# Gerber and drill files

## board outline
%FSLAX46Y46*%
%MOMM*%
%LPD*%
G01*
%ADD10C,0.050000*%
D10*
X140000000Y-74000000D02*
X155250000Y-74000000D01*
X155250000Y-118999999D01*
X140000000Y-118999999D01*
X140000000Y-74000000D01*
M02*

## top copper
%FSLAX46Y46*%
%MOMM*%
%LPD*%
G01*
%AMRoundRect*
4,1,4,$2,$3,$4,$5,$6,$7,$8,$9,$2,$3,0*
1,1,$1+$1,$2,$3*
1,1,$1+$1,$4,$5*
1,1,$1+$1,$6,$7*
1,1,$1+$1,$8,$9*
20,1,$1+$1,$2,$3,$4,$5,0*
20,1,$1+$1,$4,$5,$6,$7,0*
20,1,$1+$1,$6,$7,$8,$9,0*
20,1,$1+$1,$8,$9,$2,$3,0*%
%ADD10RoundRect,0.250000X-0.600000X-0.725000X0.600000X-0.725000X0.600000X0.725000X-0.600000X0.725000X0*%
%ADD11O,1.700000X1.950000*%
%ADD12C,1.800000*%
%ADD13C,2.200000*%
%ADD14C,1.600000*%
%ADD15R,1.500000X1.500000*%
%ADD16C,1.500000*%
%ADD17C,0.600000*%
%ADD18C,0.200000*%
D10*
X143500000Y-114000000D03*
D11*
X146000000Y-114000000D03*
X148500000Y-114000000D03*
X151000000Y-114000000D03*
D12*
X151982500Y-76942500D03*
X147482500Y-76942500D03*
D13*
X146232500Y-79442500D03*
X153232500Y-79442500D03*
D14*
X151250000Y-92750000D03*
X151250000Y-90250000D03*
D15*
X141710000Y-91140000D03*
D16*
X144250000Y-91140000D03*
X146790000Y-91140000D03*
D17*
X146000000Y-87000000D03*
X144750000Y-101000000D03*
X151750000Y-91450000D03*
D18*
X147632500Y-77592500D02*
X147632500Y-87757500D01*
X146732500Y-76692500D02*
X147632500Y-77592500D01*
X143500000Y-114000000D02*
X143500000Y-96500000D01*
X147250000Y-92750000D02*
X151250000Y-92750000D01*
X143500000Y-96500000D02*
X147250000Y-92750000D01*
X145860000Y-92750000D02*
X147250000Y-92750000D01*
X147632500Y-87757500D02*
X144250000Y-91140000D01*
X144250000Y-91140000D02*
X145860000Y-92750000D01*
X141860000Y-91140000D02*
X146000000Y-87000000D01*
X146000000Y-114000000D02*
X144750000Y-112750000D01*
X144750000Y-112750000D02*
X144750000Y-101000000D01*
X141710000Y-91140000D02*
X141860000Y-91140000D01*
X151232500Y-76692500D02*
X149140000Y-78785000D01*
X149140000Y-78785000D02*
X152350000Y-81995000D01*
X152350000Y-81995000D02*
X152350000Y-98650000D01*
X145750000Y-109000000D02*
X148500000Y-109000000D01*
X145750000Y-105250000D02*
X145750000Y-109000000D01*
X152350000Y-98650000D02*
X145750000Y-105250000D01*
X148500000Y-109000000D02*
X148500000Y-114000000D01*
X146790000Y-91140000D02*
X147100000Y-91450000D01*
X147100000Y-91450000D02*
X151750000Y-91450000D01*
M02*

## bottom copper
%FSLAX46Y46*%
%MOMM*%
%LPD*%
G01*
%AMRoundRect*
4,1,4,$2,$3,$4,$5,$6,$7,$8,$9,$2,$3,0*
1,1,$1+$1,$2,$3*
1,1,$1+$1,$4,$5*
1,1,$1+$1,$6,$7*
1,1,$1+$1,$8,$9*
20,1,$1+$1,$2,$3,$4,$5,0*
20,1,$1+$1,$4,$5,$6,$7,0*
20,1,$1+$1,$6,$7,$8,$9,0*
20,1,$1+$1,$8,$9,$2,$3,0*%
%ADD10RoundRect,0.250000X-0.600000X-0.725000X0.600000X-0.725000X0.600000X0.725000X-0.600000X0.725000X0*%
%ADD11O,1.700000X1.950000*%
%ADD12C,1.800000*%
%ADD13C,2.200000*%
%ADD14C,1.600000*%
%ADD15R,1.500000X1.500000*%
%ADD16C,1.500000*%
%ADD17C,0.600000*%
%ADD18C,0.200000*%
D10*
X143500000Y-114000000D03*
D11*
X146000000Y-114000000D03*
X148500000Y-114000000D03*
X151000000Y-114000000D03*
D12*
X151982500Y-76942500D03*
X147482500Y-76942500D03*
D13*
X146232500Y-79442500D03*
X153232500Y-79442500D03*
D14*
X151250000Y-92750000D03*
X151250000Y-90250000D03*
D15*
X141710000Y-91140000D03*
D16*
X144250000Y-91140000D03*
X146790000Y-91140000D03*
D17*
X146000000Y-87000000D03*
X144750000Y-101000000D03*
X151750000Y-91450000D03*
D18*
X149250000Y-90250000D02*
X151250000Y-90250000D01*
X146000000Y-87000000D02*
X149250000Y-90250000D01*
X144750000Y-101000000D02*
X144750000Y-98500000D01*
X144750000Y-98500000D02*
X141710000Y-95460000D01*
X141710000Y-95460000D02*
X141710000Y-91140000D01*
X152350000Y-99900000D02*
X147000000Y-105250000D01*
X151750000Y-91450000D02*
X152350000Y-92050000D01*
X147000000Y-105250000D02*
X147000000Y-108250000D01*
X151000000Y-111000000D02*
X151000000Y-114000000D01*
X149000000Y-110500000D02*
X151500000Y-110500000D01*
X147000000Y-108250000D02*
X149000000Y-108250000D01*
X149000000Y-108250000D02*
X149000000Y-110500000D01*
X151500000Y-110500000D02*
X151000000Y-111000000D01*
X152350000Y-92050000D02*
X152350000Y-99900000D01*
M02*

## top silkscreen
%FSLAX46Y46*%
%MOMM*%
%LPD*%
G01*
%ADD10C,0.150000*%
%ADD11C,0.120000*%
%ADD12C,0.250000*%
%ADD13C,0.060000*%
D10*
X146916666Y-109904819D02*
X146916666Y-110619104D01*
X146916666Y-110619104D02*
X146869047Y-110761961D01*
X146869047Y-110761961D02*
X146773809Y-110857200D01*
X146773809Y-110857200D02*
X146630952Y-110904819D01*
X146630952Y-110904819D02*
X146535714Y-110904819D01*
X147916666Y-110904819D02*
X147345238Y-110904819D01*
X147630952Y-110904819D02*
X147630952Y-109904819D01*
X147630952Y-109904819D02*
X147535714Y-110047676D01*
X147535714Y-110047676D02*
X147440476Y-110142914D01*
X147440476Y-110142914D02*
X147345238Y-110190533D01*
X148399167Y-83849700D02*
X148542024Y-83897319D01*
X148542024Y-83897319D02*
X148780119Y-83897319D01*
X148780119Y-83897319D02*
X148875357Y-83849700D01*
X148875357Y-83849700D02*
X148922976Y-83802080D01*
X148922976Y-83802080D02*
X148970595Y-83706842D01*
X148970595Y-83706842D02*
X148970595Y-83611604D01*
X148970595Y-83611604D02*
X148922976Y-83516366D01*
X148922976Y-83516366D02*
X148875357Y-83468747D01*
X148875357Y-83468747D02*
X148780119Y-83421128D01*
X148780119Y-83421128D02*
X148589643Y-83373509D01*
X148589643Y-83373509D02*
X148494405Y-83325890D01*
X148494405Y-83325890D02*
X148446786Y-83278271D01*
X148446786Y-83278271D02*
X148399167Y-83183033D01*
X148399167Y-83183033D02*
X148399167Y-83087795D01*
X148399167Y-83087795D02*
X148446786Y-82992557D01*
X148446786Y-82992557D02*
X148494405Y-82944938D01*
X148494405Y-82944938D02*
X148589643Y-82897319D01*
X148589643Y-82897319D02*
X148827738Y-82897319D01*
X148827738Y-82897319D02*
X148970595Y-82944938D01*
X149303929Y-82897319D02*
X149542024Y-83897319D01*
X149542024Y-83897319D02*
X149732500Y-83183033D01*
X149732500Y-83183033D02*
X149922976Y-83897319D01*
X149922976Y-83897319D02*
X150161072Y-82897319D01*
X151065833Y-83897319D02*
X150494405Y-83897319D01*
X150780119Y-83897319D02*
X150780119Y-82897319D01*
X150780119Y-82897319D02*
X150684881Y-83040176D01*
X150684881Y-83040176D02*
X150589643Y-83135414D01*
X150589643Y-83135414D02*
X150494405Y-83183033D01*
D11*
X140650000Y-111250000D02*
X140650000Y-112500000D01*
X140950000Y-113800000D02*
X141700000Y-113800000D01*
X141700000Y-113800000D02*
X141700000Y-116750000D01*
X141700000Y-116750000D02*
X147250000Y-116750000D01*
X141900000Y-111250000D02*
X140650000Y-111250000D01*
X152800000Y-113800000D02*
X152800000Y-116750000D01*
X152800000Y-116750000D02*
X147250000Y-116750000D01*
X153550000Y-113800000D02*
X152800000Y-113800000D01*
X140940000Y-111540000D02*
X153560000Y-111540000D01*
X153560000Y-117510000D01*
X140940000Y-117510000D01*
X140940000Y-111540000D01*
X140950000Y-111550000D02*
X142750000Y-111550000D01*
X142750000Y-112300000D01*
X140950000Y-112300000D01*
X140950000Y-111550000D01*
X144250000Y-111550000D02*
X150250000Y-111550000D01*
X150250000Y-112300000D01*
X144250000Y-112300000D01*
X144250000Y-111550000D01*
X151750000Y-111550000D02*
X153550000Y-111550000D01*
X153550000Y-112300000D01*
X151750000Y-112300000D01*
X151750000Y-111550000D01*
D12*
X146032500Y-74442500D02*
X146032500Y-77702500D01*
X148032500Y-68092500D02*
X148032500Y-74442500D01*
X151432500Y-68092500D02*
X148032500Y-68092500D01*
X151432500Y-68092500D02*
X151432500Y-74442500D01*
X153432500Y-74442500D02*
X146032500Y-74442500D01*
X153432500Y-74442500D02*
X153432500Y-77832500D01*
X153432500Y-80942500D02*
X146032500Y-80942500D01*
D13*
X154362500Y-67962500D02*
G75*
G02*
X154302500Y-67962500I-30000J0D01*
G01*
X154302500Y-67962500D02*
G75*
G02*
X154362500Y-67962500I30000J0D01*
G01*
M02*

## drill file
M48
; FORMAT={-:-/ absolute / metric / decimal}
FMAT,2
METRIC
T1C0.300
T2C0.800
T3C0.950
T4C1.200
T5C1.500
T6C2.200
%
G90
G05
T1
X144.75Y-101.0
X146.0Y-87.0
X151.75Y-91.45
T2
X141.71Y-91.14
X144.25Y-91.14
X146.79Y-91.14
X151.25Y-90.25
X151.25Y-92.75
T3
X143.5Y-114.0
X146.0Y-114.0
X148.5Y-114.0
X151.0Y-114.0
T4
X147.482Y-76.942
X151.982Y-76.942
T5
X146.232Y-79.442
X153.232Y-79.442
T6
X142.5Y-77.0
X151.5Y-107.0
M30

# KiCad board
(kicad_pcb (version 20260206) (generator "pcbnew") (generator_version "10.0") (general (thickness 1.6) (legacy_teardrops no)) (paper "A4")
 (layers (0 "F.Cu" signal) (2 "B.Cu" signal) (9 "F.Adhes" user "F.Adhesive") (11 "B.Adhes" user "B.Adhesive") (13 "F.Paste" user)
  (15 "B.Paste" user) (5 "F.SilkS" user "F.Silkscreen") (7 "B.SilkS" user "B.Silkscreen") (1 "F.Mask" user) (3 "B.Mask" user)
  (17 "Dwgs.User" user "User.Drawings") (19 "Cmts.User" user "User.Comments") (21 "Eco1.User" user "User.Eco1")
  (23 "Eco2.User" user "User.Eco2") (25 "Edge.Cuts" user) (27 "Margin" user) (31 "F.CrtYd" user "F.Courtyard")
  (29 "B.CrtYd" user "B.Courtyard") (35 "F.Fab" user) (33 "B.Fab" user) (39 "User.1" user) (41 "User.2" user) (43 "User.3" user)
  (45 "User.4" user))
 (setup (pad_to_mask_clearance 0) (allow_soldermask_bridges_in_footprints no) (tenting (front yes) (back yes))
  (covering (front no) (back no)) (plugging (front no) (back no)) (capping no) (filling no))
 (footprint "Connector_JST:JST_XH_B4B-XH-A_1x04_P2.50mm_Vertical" (layer "F.Cu") (at 143.5 114)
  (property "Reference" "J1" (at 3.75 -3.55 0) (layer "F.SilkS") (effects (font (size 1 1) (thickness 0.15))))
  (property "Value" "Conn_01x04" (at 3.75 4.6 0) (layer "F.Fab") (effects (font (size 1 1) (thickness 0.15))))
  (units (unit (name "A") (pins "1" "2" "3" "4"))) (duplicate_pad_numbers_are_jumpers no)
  (fp_line (start -2.85 -2.75) (end -2.85 -1.5) (stroke (width 0.12) (type solid)) (layer "F.SilkS"))
  (fp_line (start -2.55 -0.2) (end -1.8 -0.2) (stroke (width 0.12) (type solid)) (layer "F.SilkS"))
  (fp_line (start -1.8 -0.2) (end -1.8 2.75) (stroke (width 0.12) (type solid)) (layer "F.SilkS"))
  (fp_line (start -1.8 2.75) (end 3.75 2.75) (stroke (width 0.12) (type solid)) (layer "F.SilkS"))
  (fp_line (start -1.6 -2.75) (end -2.85 -2.75) (stroke (width 0.12) (type solid)) (layer "F.SilkS"))
  (fp_line (start 9.3 -0.2) (end 9.3 2.75) (stroke (width 0.12) (type solid)) (layer "F.SilkS"))
  (fp_line (start 9.3 2.75) (end 3.75 2.75) (stroke (width 0.12) (type solid)) (layer "F.SilkS"))
  (fp_line (start 10.05 -0.2) (end 9.3 -0.2) (stroke (width 0.12) (type solid)) (layer "F.SilkS"))
  (fp_rect (start -2.56 -2.46) (end 10.06 3.51) (stroke (width 0.12) (type solid)) (fill no) (layer "F.SilkS"))
  (fp_rect (start -2.55 -2.45) (end -0.75 -1.7) (stroke (width 0.12) (type solid)) (fill no) (layer "F.SilkS"))
  (fp_rect (start 0.75 -2.45) (end 6.75 -1.7) (stroke (width 0.12) (type solid)) (fill no) (layer "F.SilkS"))
  (fp_rect (start 8.25 -2.45) (end 10.05 -1.7) (stroke (width 0.12) (type solid)) (fill no) (layer "F.SilkS"))
  (pad "1" thru_hole roundrect (at 0 0) (size 1.7 1.95) (drill 0.95) (layers "*.Cu" "*.Mask") (remove_unused_layers no)
   (roundrect_rratio 0.147059) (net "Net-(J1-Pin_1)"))
  (pad "2" thru_hole oval (at 2.5 0) (size 1.7 1.95) (drill 0.95) (layers "*.Cu" "*.Mask") (remove_unused_layers no) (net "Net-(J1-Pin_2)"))
  (pad "3" thru_hole oval (at 5 0) (size 1.7 1.95) (drill 0.95) (layers "*.Cu" "*.Mask") (remove_unused_layers no) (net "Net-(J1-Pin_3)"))
  (pad "4" thru_hole oval (at 7.5 0) (size 1.7 1.95) (drill 0.95) (layers "*.Cu" "*.Mask") (remove_unused_layers no) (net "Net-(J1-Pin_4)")))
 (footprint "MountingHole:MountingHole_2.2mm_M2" (layer "F.Cu") (at 142.5 77)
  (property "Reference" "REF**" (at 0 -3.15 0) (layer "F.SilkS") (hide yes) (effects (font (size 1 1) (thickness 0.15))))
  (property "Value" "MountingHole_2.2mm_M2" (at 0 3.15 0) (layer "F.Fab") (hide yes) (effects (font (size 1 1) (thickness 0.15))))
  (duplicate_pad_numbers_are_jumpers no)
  (pad "" np_thru_hole circle (at 0 0) (size 2.2 2.2) (drill 2.2) (layers "*.Cu" "*.Mask")))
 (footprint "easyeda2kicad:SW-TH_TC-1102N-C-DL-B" (layer "F.Cu") (at 149.7325 78.1925 180)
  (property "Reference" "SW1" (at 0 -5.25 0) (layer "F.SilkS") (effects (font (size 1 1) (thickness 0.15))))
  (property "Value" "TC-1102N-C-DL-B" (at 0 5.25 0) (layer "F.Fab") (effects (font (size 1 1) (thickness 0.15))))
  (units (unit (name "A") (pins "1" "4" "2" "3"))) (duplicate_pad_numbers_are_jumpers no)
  (fp_line (start 3.7 3.75) (end 3.7 0.49) (stroke (width 0.25) (type solid)) (layer "F.SilkS"))
  (fp_line (start 1.7 10.1) (end 1.7 3.75) (stroke (width 0.25) (type solid)) (layer "F.SilkS"))
  (fp_line (start -1.7 10.1) (end 1.7 10.1) (stroke (width 0.25) (type solid)) (layer "F.SilkS"))
  (fp_line (start -1.7 10.1) (end -1.7 3.75) (stroke (width 0.25) (type solid)) (layer "F.SilkS"))
  (fp_line (start -3.7 3.75) (end 3.7 3.75) (stroke (width 0.25) (type solid)) (layer "F.SilkS"))
  (fp_line (start -3.7 3.75) (end -3.7 0.36) (stroke (width 0.25) (type solid)) (layer "F.SilkS"))
  (fp_line (start -3.7 -2.75) (end 3.7 -2.75) (stroke (width 0.25) (type solid)) (layer "F.SilkS"))
  (fp_circle (center -4.6 10.23) (end -4.57 10.23) (stroke (width 0.06) (type solid)) (fill no) (layer "F.SilkS"))
  (pad "1" thru_hole circle (at -2.25 1.25 180) (size 1.8 1.8) (drill 1.199998) (layers "*.Cu" "*.Mask") (remove_unused_layers no)
   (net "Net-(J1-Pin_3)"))
  (pad "2" thru_hole circle (at 2.25 1.25 180) (size 1.8 1.8) (drill 1.199998) (layers "*.Cu" "*.Mask") (remove_unused_layers no)
   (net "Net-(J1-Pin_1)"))
  (pad "3" thru_hole circle (at 3.5 -1.25 180) (size 2.2 2.2) (drill 1.500022) (layers "*.Cu" "*.Mask") (remove_unused_layers no)
   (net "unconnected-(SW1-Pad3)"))
  (pad "4" thru_hole circle (at -3.5 -1.25 180) (size 2.2 2.2) (drill 1.500022) (layers "*.Cu" "*.Mask") (remove_unused_layers no)
   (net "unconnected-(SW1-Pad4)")))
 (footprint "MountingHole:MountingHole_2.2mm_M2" (layer "F.Cu") (at 151.5 107)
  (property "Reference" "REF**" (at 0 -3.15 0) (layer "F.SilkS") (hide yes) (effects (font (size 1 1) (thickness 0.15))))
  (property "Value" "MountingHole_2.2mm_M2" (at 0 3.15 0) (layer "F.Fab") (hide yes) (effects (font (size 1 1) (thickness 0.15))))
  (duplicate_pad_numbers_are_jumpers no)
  (pad "" np_thru_hole circle (at 0 0) (size 2.2 2.2) (drill 2.2) (layers "*.Cu" "*.Mask")))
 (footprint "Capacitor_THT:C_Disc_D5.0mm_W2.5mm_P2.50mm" (layer "B.Cu") (at 151.25 92.75 90)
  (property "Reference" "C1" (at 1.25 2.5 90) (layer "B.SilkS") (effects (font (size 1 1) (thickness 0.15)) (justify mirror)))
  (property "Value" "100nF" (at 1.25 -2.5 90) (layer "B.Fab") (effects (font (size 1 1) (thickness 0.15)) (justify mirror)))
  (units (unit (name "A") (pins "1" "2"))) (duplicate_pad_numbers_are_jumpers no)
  (pad "1" thru_hole circle (at 0 0 90) (size 1.6 1.6) (drill 0.8) (layers "*.Cu" "*.Mask") (remove_unused_layers no) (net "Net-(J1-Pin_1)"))
  (pad "2" thru_hole circle (at 2.5 0 90) (size 1.6 1.6) (drill 0.8) (layers "*.Cu" "*.Mask") (remove_unused_layers no)
   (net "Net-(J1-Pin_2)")))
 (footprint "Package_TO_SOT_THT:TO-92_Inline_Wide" (layer "B.Cu") (at 141.71 91.14)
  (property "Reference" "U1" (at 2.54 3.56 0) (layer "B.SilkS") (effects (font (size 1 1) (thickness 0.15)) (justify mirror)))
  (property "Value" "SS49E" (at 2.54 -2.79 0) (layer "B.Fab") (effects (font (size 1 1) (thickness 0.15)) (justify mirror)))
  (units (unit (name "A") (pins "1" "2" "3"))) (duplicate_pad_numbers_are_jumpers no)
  (pad "1" thru_hole rect (at 0 0) (size 1.5 1.5) (drill 0.8) (layers "*.Cu" "*.Mask") (remove_unused_layers no) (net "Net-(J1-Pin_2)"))
  (pad "2" thru_hole circle (at 2.54 0) (size 1.5 1.5) (drill 0.8) (layers "*.Cu" "*.Mask") (remove_unused_layers no) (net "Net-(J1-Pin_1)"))
  (pad "3" thru_hole circle (at 5.08 0) (size 1.5 1.5) (drill 0.8) (layers "*.Cu" "*.Mask") (remove_unused_layers no) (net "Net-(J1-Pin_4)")))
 (gr_rect (start 140 74) (end 155.25 118.999999) (stroke (width 0.05) (type default)) (fill no) (layer "Edge.Cuts"))
 (segment (start 147.6325 77.5925) (end 147.6325 87.7575) (width 0.2) (layer "F.Cu") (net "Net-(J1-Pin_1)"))
 (segment (start 146.7325 76.6925) (end 147.6325 77.5925) (width 0.2) (layer "F.Cu") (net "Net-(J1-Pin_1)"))
 (segment (start 143.5 114) (end 143.5 96.5) (width 0.2) (layer "F.Cu") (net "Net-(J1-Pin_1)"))
 (segment (start 147.25 92.75) (end 151.25 92.75) (width 0.2) (layer "F.Cu") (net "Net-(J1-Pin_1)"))
 (segment (start 143.5 96.5) (end 147.25 92.75) (width 0.2) (layer "F.Cu") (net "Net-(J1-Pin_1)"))
 (segment (start 145.86 92.75) (end 147.25 92.75) (width 0.2) (layer "F.Cu") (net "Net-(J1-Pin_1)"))
 (segment (start 147.6325 87.7575) (end 144.25 91.14) (width 0.2) (layer "F.Cu") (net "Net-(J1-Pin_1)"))
 (segment (start 144.25 91.14) (end 145.86 92.75) (width 0.2) (layer "F.Cu") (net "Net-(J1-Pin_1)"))
 (segment (start 141.86 91.14) (end 146 87) (width 0.2) (layer "F.Cu") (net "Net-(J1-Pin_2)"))
 (segment (start 146 114) (end 144.75 112.75) (width 0.2) (layer "F.Cu") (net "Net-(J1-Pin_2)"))
 (segment (start 144.75 112.75) (end 144.75 101) (width 0.2) (layer "F.Cu") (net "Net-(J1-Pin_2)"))
 (segment (start 141.71 91.14) (end 141.86 91.14) (width 0.2) (layer "F.Cu") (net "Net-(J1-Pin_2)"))
 (via (at 146 87) (size 0.6) (drill 0.3) (layers "F.Cu" "B.Cu") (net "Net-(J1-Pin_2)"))
 (via (at 144.75 101) (size 0.6) (drill 0.3) (layers "F.Cu" "B.Cu") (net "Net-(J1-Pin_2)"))
 (segment (start 149.25 90.25) (end 151.25 90.25) (width 0.2) (layer "B.Cu") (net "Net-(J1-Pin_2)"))
 (segment (start 146 87) (end 149.25 90.25) (width 0.2) (layer "B.Cu") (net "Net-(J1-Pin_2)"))
 (segment (start 144.75 101) (end 144.75 98.5) (width 0.2) (layer "B.Cu") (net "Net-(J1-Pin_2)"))
 (segment (start 144.75 98.5) (end 141.71 95.46) (width 0.2) (layer "B.Cu") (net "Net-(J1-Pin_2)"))
 (segment (start 141.71 95.46) (end 141.71 91.14) (width 0.2) (layer "B.Cu") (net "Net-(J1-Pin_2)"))
 (segment (start 151.2325 76.6925) (end 149.14 78.785) (width 0.2) (layer "F.Cu") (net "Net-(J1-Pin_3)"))
 (segment (start 149.14 78.785) (end 152.35 81.995) (width 0.2) (layer "F.Cu") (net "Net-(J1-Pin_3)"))
 (segment (start 152.35 81.995) (end 152.35 98.65) (width 0.2) (layer "F.Cu") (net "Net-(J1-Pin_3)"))
 (segment (start 145.75 109) (end 148.5 109) (width 0.2) (layer "F.Cu") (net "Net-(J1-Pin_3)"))
 (segment (start 145.75 105.25) (end 145.75 109) (width 0.2) (layer "F.Cu") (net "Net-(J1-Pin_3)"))
 (segment (start 152.35 98.65) (end 145.75 105.25) (width 0.2) (layer "F.Cu") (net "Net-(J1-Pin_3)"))
 (segment (start 148.5 109) (end 148.5 114) (width 0.2) (layer "F.Cu") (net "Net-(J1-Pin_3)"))
 (segment (start 146.79 91.14) (end 147.1 91.45) (width 0.2) (layer "F.Cu") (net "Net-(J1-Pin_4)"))
 (segment (start 147.1 91.45) (end 151.75 91.45) (width 0.2) (layer "F.Cu") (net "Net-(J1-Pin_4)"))
 (via (at 151.75 91.45) (size 0.6) (drill 0.3) (layers "F.Cu" "B.Cu") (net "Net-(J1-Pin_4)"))
 (segment (start 152.35 99.9) (end 147 105.25) (width 0.2) (layer "B.Cu") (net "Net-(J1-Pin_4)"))
 (segment (start 151.75 91.45) (end 152.35 92.05) (width 0.2) (layer "B.Cu") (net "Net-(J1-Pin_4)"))
 (segment (start 147 105.25) (end 147 108.25) (width 0.2) (layer "B.Cu") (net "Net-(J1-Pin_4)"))
 (segment (start 151 111) (end 151 114) (width 0.2) (layer "B.Cu") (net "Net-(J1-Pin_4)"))
 (segment (start 149 110.5) (end 151.5 110.5) (width 0.2) (layer "B.Cu") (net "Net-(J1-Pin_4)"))
 (segment (start 147 108.25) (end 149 108.25) (width 0.2) (layer "B.Cu") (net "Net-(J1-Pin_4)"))
 (segment (start 149 108.25) (end 149 110.5) (width 0.2) (layer "B.Cu") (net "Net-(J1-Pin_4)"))
 (segment (start 151.5 110.5) (end 151 111) (width 0.2) (layer "B.Cu") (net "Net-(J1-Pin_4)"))
 (segment (start 152.35 92.05) (end 152.35 99.9) (width 0.2) (layer "B.Cu") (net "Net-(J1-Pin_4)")))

